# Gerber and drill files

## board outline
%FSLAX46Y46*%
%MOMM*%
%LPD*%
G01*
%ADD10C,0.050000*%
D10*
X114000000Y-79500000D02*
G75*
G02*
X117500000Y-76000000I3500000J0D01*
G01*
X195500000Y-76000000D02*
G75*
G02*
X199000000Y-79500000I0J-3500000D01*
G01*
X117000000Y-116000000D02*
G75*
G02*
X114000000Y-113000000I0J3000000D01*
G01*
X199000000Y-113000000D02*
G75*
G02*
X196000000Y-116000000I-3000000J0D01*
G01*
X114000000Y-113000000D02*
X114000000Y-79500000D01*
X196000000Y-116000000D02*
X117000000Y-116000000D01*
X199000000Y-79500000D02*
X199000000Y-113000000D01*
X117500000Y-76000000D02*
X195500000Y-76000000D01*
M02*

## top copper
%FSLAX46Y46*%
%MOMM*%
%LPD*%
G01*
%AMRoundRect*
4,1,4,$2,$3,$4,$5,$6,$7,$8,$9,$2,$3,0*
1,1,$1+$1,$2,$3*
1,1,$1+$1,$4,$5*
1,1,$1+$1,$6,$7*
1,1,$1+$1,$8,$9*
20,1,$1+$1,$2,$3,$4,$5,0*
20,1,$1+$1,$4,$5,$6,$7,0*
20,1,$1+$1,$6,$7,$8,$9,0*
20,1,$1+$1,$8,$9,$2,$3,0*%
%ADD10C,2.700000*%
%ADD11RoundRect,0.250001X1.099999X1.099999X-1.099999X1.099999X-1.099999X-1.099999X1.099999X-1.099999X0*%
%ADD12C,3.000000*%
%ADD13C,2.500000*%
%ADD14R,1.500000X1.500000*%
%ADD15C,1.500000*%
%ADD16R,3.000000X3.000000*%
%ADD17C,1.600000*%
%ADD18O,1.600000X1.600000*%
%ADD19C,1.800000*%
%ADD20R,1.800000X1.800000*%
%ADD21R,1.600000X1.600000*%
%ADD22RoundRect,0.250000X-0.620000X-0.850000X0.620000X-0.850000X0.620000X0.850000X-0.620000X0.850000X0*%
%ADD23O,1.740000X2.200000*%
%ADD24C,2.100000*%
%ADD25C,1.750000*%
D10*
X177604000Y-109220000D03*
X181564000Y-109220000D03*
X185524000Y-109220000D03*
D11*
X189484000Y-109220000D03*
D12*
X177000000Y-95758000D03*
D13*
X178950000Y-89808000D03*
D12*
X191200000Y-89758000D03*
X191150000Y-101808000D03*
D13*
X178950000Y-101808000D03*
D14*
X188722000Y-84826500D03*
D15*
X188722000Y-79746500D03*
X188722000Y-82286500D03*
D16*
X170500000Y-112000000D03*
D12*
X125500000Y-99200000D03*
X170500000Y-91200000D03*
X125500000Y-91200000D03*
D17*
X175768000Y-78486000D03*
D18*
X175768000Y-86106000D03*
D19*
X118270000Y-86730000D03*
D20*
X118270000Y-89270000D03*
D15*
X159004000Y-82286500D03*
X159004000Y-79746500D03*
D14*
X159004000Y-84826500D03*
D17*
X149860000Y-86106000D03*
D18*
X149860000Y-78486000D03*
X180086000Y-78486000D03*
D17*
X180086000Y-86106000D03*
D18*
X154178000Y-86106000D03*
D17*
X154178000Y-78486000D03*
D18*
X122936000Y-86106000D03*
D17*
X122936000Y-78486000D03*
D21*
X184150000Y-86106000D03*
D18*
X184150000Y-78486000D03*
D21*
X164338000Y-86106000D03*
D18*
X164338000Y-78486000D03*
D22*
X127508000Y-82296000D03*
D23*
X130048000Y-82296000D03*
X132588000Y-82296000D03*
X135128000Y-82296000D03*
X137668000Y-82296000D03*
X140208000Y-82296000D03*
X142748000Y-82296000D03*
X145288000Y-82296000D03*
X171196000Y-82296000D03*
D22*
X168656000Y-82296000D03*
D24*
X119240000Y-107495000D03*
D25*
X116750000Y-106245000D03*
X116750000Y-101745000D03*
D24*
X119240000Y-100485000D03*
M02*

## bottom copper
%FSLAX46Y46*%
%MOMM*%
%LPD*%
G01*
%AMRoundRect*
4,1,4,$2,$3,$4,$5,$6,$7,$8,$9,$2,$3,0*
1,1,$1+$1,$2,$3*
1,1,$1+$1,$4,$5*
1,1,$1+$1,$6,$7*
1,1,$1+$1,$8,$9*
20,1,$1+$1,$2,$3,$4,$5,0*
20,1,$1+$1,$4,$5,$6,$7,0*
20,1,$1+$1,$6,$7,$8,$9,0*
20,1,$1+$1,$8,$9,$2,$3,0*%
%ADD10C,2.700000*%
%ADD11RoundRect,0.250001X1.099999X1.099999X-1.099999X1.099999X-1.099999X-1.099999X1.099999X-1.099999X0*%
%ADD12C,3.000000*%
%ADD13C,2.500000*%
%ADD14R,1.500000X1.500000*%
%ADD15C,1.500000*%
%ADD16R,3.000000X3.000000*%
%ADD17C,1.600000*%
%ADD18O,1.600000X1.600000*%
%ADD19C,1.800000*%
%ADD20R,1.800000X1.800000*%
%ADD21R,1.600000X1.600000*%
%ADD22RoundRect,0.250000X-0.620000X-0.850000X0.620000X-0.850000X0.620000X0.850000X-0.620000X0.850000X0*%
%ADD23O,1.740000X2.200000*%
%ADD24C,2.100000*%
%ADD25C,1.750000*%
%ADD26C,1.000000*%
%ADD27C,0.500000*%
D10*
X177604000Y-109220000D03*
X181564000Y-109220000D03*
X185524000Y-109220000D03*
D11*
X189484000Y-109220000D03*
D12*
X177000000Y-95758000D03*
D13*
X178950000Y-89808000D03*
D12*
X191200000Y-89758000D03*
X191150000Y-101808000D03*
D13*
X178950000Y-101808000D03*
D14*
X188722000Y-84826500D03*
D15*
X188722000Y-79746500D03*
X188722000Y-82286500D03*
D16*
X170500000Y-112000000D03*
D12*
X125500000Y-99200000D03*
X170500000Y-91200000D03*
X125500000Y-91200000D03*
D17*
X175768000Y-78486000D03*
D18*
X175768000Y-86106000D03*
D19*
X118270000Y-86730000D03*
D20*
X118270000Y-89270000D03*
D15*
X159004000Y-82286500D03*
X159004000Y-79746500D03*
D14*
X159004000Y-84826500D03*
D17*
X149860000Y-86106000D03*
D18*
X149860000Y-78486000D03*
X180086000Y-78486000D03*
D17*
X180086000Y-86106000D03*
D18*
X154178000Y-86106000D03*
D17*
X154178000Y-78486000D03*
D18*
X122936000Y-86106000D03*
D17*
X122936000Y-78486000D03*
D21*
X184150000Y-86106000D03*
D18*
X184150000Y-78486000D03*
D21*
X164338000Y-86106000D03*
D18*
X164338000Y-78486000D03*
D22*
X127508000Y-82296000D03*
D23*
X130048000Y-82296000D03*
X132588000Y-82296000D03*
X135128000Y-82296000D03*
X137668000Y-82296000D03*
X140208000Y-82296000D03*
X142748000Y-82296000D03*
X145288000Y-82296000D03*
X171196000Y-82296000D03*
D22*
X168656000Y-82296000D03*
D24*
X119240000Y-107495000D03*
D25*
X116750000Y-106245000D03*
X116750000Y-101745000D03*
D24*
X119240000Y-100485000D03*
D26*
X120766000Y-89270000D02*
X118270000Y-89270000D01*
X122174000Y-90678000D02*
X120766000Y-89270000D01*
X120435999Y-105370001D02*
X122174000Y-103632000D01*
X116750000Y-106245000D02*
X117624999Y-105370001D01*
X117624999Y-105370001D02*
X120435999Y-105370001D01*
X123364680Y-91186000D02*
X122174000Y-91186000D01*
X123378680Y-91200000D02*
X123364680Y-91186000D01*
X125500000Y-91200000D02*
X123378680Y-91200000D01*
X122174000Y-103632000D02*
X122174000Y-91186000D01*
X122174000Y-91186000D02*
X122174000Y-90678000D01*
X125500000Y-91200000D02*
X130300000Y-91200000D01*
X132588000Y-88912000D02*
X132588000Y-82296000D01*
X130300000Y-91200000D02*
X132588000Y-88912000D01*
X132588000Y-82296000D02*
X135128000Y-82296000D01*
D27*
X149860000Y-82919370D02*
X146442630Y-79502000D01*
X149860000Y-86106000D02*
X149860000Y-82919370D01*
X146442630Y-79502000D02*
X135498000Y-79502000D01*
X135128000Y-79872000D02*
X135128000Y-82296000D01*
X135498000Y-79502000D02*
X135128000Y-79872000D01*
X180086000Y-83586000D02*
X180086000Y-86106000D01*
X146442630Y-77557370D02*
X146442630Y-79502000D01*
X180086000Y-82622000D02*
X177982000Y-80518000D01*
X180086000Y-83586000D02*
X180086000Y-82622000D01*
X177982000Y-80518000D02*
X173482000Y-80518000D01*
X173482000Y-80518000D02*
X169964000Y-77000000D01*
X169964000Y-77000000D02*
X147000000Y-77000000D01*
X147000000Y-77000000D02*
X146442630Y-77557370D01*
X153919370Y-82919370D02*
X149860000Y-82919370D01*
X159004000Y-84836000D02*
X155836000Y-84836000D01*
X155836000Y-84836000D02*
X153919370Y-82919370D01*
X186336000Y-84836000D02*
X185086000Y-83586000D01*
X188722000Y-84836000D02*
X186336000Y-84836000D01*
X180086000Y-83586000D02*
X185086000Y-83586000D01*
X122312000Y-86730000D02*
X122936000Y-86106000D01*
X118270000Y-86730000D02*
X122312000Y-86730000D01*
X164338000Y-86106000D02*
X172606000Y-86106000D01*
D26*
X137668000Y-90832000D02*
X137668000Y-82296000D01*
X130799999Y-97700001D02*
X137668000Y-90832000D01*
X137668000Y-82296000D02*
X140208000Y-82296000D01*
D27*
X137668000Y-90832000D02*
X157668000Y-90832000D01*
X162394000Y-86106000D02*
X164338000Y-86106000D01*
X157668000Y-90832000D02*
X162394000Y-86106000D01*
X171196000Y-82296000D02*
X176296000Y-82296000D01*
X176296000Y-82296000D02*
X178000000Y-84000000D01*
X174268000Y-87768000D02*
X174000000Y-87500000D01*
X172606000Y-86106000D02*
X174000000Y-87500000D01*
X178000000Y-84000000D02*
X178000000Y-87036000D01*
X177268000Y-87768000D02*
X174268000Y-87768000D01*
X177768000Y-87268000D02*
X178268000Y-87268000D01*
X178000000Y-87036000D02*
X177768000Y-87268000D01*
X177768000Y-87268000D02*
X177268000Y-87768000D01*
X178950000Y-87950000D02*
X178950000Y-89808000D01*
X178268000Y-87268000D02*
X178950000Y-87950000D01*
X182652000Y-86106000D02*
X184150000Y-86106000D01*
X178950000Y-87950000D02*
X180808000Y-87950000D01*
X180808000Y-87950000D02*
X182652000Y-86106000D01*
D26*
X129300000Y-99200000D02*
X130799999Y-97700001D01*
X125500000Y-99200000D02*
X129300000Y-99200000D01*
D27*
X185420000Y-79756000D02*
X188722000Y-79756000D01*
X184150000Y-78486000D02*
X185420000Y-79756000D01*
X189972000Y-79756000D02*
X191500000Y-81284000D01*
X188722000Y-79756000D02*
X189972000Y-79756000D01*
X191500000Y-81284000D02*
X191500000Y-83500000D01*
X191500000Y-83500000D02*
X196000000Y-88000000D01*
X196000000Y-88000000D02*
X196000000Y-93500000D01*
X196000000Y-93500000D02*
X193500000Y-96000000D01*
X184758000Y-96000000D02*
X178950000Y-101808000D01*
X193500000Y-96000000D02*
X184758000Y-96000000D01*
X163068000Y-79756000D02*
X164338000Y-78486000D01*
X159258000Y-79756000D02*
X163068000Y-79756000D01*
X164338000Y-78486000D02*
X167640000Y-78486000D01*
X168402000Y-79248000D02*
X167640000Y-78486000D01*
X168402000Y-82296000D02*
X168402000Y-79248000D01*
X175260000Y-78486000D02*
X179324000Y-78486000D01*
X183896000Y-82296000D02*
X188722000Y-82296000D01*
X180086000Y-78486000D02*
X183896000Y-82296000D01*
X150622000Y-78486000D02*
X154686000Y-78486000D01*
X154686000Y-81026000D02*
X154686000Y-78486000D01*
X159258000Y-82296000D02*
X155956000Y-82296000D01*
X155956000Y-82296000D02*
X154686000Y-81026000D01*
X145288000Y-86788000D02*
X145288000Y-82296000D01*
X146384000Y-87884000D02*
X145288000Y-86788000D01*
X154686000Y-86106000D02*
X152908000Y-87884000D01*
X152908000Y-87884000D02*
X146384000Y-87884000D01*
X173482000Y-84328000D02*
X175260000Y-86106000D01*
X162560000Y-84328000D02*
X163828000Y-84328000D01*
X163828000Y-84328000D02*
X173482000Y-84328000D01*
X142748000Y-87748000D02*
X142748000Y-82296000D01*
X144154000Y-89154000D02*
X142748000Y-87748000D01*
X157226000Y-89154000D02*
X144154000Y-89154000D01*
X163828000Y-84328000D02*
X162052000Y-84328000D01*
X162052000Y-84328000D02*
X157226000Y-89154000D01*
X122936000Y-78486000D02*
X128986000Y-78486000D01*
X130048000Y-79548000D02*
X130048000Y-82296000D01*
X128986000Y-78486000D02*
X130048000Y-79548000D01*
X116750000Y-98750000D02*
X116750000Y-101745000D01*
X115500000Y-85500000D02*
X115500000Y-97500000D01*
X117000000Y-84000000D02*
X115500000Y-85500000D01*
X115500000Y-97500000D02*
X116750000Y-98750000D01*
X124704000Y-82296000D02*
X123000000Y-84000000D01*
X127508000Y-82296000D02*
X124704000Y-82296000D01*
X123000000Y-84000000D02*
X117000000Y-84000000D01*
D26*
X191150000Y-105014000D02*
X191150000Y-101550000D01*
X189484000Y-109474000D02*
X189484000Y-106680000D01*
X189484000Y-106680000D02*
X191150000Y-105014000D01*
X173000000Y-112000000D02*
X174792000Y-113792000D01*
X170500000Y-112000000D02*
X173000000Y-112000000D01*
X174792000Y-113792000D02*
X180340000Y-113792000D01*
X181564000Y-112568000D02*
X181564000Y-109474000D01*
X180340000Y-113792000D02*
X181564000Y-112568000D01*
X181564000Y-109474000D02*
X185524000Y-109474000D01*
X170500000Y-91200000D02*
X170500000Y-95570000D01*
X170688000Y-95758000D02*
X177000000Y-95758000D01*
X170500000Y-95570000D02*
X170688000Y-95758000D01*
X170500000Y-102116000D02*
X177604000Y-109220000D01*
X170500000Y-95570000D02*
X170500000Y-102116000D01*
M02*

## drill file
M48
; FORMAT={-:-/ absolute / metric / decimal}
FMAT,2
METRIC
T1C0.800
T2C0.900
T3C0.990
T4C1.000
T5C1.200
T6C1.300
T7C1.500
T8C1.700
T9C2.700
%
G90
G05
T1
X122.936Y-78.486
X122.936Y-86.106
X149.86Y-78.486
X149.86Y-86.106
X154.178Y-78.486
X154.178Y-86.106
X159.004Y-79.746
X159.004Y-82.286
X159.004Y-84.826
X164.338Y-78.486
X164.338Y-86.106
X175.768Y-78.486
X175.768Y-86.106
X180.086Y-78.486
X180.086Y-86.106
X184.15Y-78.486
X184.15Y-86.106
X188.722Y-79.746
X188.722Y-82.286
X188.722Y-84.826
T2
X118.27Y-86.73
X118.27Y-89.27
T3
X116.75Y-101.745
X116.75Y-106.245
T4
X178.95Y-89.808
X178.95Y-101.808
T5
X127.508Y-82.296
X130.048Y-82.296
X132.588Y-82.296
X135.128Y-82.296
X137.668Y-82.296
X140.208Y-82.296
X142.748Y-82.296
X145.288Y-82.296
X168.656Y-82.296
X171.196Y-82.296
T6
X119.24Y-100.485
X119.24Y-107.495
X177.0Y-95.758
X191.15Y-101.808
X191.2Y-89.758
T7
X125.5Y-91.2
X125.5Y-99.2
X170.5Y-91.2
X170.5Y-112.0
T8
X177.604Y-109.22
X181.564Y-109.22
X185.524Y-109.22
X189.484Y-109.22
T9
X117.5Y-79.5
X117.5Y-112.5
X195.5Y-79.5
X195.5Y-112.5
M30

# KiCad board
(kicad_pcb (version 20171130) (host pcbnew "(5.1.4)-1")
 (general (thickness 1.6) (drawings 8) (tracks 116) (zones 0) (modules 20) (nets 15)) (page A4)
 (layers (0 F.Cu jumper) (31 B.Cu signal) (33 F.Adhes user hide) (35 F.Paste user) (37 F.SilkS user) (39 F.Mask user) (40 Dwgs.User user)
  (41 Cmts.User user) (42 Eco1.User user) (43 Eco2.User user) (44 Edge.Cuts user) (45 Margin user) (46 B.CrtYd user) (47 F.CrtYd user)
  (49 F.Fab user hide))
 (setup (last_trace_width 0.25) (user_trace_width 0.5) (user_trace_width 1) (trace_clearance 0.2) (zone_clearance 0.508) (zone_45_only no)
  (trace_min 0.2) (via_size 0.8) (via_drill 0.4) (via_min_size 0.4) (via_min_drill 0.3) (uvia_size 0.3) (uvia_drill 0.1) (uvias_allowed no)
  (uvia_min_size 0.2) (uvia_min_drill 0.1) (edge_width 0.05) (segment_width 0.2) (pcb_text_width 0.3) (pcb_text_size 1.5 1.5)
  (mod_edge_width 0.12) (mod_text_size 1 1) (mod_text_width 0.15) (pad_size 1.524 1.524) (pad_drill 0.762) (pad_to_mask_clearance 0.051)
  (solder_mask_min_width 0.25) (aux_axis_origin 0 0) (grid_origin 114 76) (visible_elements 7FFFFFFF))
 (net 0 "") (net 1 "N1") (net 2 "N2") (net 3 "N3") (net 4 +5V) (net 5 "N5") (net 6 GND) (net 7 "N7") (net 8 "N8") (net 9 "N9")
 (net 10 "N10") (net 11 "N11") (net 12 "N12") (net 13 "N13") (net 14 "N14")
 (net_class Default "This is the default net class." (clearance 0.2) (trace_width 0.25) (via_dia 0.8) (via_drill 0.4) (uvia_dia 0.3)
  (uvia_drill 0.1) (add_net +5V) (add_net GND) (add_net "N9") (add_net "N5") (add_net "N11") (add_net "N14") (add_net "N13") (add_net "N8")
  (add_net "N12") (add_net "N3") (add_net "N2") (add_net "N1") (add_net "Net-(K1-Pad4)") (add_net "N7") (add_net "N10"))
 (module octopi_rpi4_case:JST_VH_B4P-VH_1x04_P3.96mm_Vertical (layer F.Cu) (at 189.484 109.22 180)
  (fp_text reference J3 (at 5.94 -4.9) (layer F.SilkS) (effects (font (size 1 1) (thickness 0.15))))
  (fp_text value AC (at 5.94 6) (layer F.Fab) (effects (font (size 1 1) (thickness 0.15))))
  (pad 4 thru_hole circle (at 11.88 0 180) (size 2.7 2.7) (drill 1.7) (layers *.Cu *.Mask) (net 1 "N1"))
  (pad 3 thru_hole circle (at 7.92 0 180) (size 2.7 2.7) (drill 1.7) (layers *.Cu *.Mask) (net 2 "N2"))
  (pad 2 thru_hole circle (at 3.96 0 180) (size 2.7 2.7) (drill 1.7) (layers *.Cu *.Mask) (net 2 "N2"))
  (pad 1 thru_hole roundrect (at 0 0 180) (size 2.7 2.7) (drill 1.7) (layers *.Cu *.Mask) (roundrect_rratio 0.09259299999999999)
   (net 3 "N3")))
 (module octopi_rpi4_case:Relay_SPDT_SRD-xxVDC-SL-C (layer F.Cu) (at 177 95.758)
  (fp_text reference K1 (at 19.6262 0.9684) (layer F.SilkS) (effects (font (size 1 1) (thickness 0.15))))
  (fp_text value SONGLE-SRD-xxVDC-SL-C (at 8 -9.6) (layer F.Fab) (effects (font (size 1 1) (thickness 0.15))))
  (pad 1 thru_hole circle (at 0 0 90) (size 3 3) (drill 1.3) (layers *.Cu *.Mask) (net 1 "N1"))
  (pad 5 thru_hole circle (at 1.95 -5.95 90) (size 2.5 2.5) (drill 1) (layers *.Cu *.Mask) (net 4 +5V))
  (pad 4 thru_hole circle (at 14.2 -6 90) (size 3 3) (drill 1.3) (layers *.Cu *.Mask))
  (pad 3 thru_hole circle (at 14.15 6.05 90) (size 3 3) (drill 1.3) (layers *.Cu *.Mask) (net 3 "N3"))
  (pad 2 thru_hole circle (at 1.95 6.05 90) (size 2.5 2.5) (drill 1) (layers *.Cu *.Mask) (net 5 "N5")))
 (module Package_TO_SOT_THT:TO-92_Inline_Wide (layer F.Cu) (at 188.722 84.8265 90)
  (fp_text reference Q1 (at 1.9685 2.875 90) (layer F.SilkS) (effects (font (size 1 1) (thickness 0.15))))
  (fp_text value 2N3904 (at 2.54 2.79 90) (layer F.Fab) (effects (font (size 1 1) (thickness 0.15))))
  (pad 1 thru_hole rect (at 0 0 180) (size 1.5 1.5) (drill 0.8) (layers *.Cu *.Mask) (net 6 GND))
  (pad 3 thru_hole circle (at 5.08 0 180) (size 1.5 1.5) (drill 0.8) (layers *.Cu *.Mask) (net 5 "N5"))
  (pad 2 thru_hole circle (at 2.54 0 180) (size 1.5 1.5) (drill 0.8) (layers *.Cu *.Mask) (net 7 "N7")))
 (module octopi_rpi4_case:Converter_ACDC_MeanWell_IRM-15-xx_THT (layer F.Cu) (at 170.5 112 180)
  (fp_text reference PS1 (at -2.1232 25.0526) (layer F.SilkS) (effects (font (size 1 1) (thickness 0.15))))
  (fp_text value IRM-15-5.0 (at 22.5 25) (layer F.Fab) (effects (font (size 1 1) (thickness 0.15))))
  (pad 1 thru_hole rect (at 0 0 180) (size 3 3) (drill 1.5) (layers *.Cu *.Mask) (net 2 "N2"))
  (pad 4 thru_hole circle (at 45 12.8 180) (size 3 3) (drill 1.5) (layers *.Cu *.Mask) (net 4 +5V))
  (pad 2 thru_hole circle (at 0 20.8 180) (size 3 3) (drill 1.5) (layers *.Cu *.Mask) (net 1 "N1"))
  (pad 3 thru_hole circle (at 45 20.8 180) (size 3 3) (drill 1.5) (layers *.Cu *.Mask) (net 6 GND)))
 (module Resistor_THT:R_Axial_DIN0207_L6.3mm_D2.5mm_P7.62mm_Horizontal (layer F.Cu) (at 175.768 78.486 270)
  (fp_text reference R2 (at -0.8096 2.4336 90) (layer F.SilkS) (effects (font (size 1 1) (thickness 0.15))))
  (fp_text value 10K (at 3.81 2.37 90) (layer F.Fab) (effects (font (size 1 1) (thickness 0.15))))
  (pad 1 thru_hole circle (at 0 0 270) (size 1.6 1.6) (drill 0.8) (layers *.Cu *.Mask) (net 7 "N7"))
  (pad 2 thru_hole oval (at 7.62 0 270) (size 1.6 1.6) (drill 0.8) (layers *.Cu *.Mask) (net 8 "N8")))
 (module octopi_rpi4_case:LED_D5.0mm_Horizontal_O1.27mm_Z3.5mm (layer F.Cu) (at 118.27 86.73 270)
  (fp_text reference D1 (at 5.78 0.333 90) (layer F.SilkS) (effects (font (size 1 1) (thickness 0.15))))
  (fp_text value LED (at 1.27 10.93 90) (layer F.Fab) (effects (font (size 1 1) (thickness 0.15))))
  (pad 2 thru_hole circle (at 0 0 270) (size 1.8 1.8) (drill 0.9) (layers *.Cu *.Mask) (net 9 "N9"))
  (pad 1 thru_hole rect (at 2.54 0 270) (size 1.8 1.8) (drill 0.9) (layers *.Cu *.Mask) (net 6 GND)))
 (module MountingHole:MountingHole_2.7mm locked (layer F.Cu) (at 195.5 79.5)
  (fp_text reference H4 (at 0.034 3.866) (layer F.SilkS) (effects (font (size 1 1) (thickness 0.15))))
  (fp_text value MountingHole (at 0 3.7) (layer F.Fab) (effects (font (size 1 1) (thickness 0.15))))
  (pad 1 np_thru_hole circle (at 0 0) (size 2.7 2.7) (drill 2.7) (layers *.Cu *.Mask)))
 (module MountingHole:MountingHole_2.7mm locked (layer F.Cu) (at 117.5 79.5)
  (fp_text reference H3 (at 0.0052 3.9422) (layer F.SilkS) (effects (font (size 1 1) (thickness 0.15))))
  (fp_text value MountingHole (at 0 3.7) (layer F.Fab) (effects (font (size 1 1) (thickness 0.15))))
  (pad 1 np_thru_hole circle (at 0 0) (size 2.7 2.7) (drill 2.7) (layers *.Cu *.Mask)))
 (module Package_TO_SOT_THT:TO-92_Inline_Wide (layer F.Cu) (at 159.004 84.8265 90)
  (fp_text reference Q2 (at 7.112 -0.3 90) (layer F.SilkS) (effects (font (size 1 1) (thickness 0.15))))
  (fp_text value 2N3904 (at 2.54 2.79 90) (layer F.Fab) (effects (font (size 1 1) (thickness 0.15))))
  (pad 2 thru_hole circle (at 2.54 0 180) (size 1.5 1.5) (drill 0.8) (layers *.Cu *.Mask) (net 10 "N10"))
  (pad 3 thru_hole circle (at 5.08 0 180) (size 1.5 1.5) (drill 0.8) (layers *.Cu *.Mask) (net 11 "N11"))
  (pad 1 thru_hole rect (at 0 0 180) (size 1.5 1.5) (drill 0.8) (layers *.Cu *.Mask) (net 6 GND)))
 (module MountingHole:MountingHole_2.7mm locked (layer F.Cu) (at 195.5 112.5)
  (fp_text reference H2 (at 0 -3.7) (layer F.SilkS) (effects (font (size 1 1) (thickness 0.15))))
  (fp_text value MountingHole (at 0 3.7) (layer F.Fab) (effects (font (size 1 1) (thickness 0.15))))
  (pad 1 np_thru_hole circle (at 0 0) (size 2.7 2.7) (drill 2.7) (layers *.Cu *.Mask)))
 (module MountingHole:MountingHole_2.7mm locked (layer F.Cu) (at 117.5 112.5)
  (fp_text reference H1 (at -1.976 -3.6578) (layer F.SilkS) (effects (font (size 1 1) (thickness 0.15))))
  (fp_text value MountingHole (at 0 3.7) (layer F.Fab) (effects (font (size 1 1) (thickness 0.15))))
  (pad 1 np_thru_hole circle (at 0 0) (size 2.7 2.7) (drill 2.7) (layers *.Cu *.Mask)))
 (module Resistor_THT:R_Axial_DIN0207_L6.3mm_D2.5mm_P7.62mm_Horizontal (layer F.Cu) (at 149.86 86.106 90)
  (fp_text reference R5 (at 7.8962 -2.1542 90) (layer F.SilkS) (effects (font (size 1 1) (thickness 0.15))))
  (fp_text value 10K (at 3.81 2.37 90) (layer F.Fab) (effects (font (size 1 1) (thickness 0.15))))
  (pad 1 thru_hole circle (at 0 0 90) (size 1.6 1.6) (drill 0.8) (layers *.Cu *.Mask) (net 6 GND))
  (pad 2 thru_hole oval (at 7.62 0 90) (size 1.6 1.6) (drill 0.8) (layers *.Cu *.Mask) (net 10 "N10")))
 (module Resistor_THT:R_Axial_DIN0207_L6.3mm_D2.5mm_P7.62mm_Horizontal (layer F.Cu) (at 180.086 86.106 90)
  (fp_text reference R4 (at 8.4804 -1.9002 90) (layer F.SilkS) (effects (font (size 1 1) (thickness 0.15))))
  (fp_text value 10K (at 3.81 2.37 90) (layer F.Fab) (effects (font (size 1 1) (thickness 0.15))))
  (pad 2 thru_hole oval (at 7.62 0 90) (size 1.6 1.6) (drill 0.8) (layers *.Cu *.Mask) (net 7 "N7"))
  (pad 1 thru_hole circle (at 0 0 90) (size 1.6 1.6) (drill 0.8) (layers *.Cu *.Mask) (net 6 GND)))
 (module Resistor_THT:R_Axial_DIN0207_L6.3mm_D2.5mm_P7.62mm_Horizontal (layer F.Cu) (at 154.178 78.486 270)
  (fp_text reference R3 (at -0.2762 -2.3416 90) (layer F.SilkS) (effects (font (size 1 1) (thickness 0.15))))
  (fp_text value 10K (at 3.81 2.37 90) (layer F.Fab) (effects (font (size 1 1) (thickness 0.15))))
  (pad 2 thru_hole oval (at 7.62 0 270) (size 1.6 1.6) (drill 0.8) (layers *.Cu *.Mask) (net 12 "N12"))
  (pad 1 thru_hole circle (at 0 0 270) (size 1.6 1.6) (drill 0.8) (layers *.Cu *.Mask) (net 10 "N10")))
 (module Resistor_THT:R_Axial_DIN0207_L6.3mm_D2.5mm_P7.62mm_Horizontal (layer F.Cu) (at 122.936 78.486 270)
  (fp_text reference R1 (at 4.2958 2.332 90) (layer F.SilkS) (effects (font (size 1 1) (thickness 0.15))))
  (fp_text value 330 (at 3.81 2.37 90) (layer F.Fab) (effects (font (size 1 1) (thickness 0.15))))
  (pad 2 thru_hole oval (at 7.62 0 270) (size 1.6 1.6) (drill 0.8) (layers *.Cu *.Mask) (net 9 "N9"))
  (pad 1 thru_hole circle (at 0 0 270) (size 1.6 1.6) (drill 0.8) (layers *.Cu *.Mask) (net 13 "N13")))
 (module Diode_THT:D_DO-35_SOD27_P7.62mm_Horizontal (layer F.Cu) (at 184.15 86.106 90)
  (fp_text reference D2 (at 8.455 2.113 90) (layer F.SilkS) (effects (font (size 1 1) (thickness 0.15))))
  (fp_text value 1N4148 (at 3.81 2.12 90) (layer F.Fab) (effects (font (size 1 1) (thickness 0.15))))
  (pad 1 thru_hole rect (at 0 0 90) (size 1.6 1.6) (drill 0.8) (layers *.Cu *.Mask) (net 4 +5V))
  (pad 2 thru_hole oval (at 7.62 0 90) (size 1.6 1.6) (drill 0.8) (layers *.Cu *.Mask) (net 5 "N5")))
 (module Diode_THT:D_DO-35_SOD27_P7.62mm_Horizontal (layer F.Cu) (at 164.338 86.106 90)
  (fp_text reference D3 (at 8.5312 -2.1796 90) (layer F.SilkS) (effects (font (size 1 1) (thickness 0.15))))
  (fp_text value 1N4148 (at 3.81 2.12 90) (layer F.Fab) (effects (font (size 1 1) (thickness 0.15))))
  (pad 1 thru_hole rect (at 0 0 90) (size 1.6 1.6) (drill 0.8) (layers *.Cu *.Mask) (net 4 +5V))
  (pad 2 thru_hole oval (at 7.62 0 90) (size 1.6 1.6) (drill 0.8) (layers *.Cu *.Mask) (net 11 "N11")))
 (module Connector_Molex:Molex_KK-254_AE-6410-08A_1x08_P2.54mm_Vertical (layer F.Cu) (at 127.508 82.296)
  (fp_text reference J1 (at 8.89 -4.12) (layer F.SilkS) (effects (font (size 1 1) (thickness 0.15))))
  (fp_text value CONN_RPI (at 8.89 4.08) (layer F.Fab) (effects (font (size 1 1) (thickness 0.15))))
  (pad 1 thru_hole roundrect (at 0 0) (size 1.74 2.2) (drill 1.2) (layers *.Cu *.Mask) (roundrect_rratio 0.143678) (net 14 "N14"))
  (pad 2 thru_hole oval (at 2.54 0) (size 1.74 2.2) (drill 1.2) (layers *.Cu *.Mask) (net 13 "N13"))
  (pad 3 thru_hole oval (at 5.08 0) (size 1.74 2.2) (drill 1.2) (layers *.Cu *.Mask) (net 6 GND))
  (pad 4 thru_hole oval (at 7.62 0) (size 1.74 2.2) (drill 1.2) (layers *.Cu *.Mask) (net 6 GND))
  (pad 5 thru_hole oval (at 10.16 0) (size 1.74 2.2) (drill 1.2) (layers *.Cu *.Mask) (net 4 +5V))
  (pad 6 thru_hole oval (at 12.7 0) (size 1.74 2.2) (drill 1.2) (layers *.Cu *.Mask) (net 4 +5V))
  (pad 7 thru_hole oval (at 15.24 0) (size 1.74 2.2) (drill 1.2) (layers *.Cu *.Mask) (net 8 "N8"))
  (pad 8 thru_hole oval (at 17.78 0) (size 1.74 2.2) (drill 1.2) (layers *.Cu *.Mask) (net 12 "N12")))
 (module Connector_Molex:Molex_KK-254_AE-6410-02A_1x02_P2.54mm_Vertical (layer F.Cu) (at 168.656 82.296)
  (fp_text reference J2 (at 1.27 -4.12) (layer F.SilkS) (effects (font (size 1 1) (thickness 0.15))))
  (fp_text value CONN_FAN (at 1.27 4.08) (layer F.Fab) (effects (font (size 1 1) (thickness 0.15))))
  (pad 2 thru_hole oval (at 2.54 0) (size 1.74 2.2) (drill 1.2) (layers *.Cu *.Mask) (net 4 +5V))
  (pad 1 thru_hole roundrect (at 0 0) (size 1.74 2.2) (drill 1.2) (layers *.Cu *.Mask) (roundrect_rratio 0.143678) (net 11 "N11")))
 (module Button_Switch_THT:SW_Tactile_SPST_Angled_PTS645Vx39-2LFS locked (layer F.Cu) (at 116.75 106.245 90)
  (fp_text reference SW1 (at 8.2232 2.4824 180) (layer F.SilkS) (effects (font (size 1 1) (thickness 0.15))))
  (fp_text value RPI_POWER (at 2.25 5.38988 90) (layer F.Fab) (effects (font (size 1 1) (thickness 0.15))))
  (pad "" thru_hole circle (at -1.25 2.49 90) (size 2.1 2.1) (drill 1.3) (layers *.Cu *.Mask))
  (pad 1 thru_hole circle (at 0 0 90) (size 1.75 1.75) (drill 0.99) (layers *.Cu *.Mask) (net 6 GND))
  (pad 2 thru_hole circle (at 4.5 0 90) (size 1.75 1.75) (drill 0.99) (layers *.Cu *.Mask) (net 14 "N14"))
  (pad "" thru_hole circle (at 5.76 2.49 90) (size 2.1 2.1) (drill 1.3) (layers *.Cu *.Mask)))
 (gr_arc (start 117.5 79.5) (end 117.5 76) (angle -90) (layer Edge.Cuts) (width 0.05))
 (gr_arc (start 195.5 79.5) (end 199 79.5) (angle -90) (layer Edge.Cuts) (width 0.05))
 (gr_arc (start 117 113) (end 114 113) (angle -90) (layer Edge.Cuts) (width 0.05))
 (gr_arc (start 196 113) (end 196 116) (angle -90) (layer Edge.Cuts) (width 0.05))
 (gr_line (start 114 113) (end 114 79.5) (layer Edge.Cuts) (width 0.05))
 (gr_line (start 196 116) (end 117 116) (layer Edge.Cuts) (width 0.05))
 (gr_line (start 199 79.5) (end 199 113) (layer Edge.Cuts) (width 0.05))
 (gr_line (start 117.5 76) (end 195.5 76) (layer Edge.Cuts) (width 0.05))
 (segment (start 120.766 89.27) (end 118.27 89.27) (width 1) (layer B.Cu) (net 6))
 (segment (start 122.174 90.678) (end 120.766 89.27) (width 1) (layer B.Cu) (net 6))
 (segment (start 120.435999 105.370001) (end 122.174 103.632) (width 1) (layer B.Cu) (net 6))
 (segment (start 116.75 106.245) (end 117.624999 105.370001) (width 1) (layer B.Cu) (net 6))
 (segment (start 117.624999 105.370001) (end 120.435999 105.370001) (width 1) (layer B.Cu) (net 6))
 (segment (start 123.36468 91.186) (end 122.174 91.186) (width 1) (layer B.Cu) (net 6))
 (segment (start 123.37868 91.2) (end 123.36468 91.186) (width 1) (layer B.Cu) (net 6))
 (segment (start 125.5 91.2) (end 123.37868 91.2) (width 1) (layer B.Cu) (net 6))
 (segment (start 122.174 103.632) (end 122.174 91.186) (width 1) (layer B.Cu) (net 6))
 (segment (start 122.174 91.186) (end 122.174 90.678) (width 1) (layer B.Cu) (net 6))
 (segment (start 125.5 91.2) (end 130.3 91.2) (width 1) (layer B.Cu) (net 6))
 (segment (start 132.588 88.912) (end 132.588 82.296) (width 1) (layer B.Cu) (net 6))
 (segment (start 130.3 91.2) (end 132.588 88.912) (width 1) (layer B.Cu) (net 6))
 (segment (start 132.588 82.296) (end 135.128 82.296) (width 1) (layer B.Cu) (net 6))
 (segment (start 149.86 82.91937) (end 146.44263 79.502) (width 0.5) (layer B.Cu) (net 6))
 (segment (start 149.86 86.106) (end 149.86 82.91937) (width 0.5) (layer B.Cu) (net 6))
 (segment (start 146.44263 79.502) (end 135.498 79.502) (width 0.5) (layer B.Cu) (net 6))
 (segment (start 135.128 79.872) (end 135.128 82.296) (width 0.5) (layer B.Cu) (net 6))
 (segment (start 135.498 79.502) (end 135.128 79.872) (width 0.5) (layer B.Cu) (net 6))
 (segment (start 180.086 83.586) (end 180.086 86.106) (width 0.5) (layer B.Cu) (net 6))
 (segment (start 146.44263 77.55737) (end 146.44263 79.502) (width 0.5) (layer B.Cu) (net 6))
 (segment (start 180.086 82.622) (end 177.982 80.518) (width 0.5) (layer B.Cu) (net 6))
 (segment (start 180.086 83.586) (end 180.086 82.622) (width 0.5) (layer B.Cu) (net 6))
 (segment (start 177.982 80.518) (end 173.482 80.518) (width 0.5) (layer B.Cu) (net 6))
 (segment (start 173.482 80.518) (end 169.964 77) (width 0.5) (layer B.Cu) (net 6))
 (segment (start 169.964 77) (end 147 77) (width 0.5) (layer B.Cu) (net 6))
 (segment (start 147 77) (end 146.44263 77.55737) (width 0.5) (layer B.Cu) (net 6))
 (segment (start 153.91937 82.91937) (end 149.86 82.91937) (width 0.5) (layer B.Cu) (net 6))
 (segment (start 159.004 84.836) (end 155.836 84.836) (width 0.5) (layer B.Cu) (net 6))
 (segment (start 155.836 84.836) (end 153.91937 82.91937) (width 0.5) (layer B.Cu) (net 6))
 (segment (start 186.336 84.836) (end 185.086 83.586) (width 0.5) (layer B.Cu) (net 6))
 (segment (start 188.722 84.836) (end 186.336 84.836) (width 0.5) (layer B.Cu) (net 6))
 (segment (start 180.086 83.586) (end 185.086 83.586) (width 0.5) (layer B.Cu) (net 6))
 (segment (start 122.312 86.73) (end 122.936 86.106) (width 0.5) (layer B.Cu) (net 9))
 (segment (start 118.27 86.73) (end 122.312 86.73) (width 0.5) (layer B.Cu) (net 9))
 (segment (start 164.338 86.106) (end 172.606 86.106) (width 0.5) (layer B.Cu) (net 4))
 (segment (start 137.668 90.832) (end 137.668 82.296) (width 1) (layer B.Cu) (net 4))
 (segment (start 130.799999 97.700001) (end 137.668 90.832) (width 1) (layer B.Cu) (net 4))
 (segment (start 137.668 82.296) (end 140.208 82.296) (width 1) (layer B.Cu) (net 4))
 (segment (start 137.668 90.832) (end 157.668 90.832) (width 0.5) (layer B.Cu) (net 4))
 (segment (start 162.394 86.106) (end 164.338 86.106) (width 0.5) (layer B.Cu) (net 4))
 (segment (start 157.668 90.832) (end 162.394 86.106) (width 0.5) (layer B.Cu) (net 4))
 (segment (start 171.196 82.296) (end 176.296 82.296) (width 0.5) (layer B.Cu) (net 4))
 (segment (start 176.296 82.296) (end 178 84) (width 0.5) (layer B.Cu) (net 4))
 (segment (start 174.268 87.768) (end 174 87.5) (width 0.5) (layer B.Cu) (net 4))
 (segment (start 172.606 86.106) (end 174 87.5) (width 0.5) (layer B.Cu) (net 4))
 (segment (start 178 84) (end 178 87.036) (width 0.5) (layer B.Cu) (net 4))
 (segment (start 177.268 87.768) (end 174.268 87.768) (width 0.5) (layer B.Cu) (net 4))
 (segment (start 177.768 87.268) (end 178.268 87.268) (width 0.5) (layer B.Cu) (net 4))
 (segment (start 178 87.036) (end 177.768 87.268) (width 0.5) (layer B.Cu) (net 4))
 (segment (start 177.768 87.268) (end 177.268 87.768) (width 0.5) (layer B.Cu) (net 4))
 (segment (start 178.95 87.95) (end 178.95 89.808) (width 0.5) (layer B.Cu) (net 4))
 (segment (start 178.268 87.268) (end 178.95 87.95) (width 0.5) (layer B.Cu) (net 4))
 (segment (start 182.652 86.106) (end 184.15 86.106) (width 0.5) (layer B.Cu) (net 4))
 (segment (start 178.95 87.95) (end 180.808 87.95) (width 0.5) (layer B.Cu) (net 4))
 (segment (start 180.808 87.95) (end 182.652 86.106) (width 0.5) (layer B.Cu) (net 4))
 (segment (start 129.3 99.2) (end 130.799999 97.700001) (width 1) (layer B.Cu) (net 4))
 (segment (start 125.5 99.2) (end 129.3 99.2) (width 1) (layer B.Cu) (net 4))
 (segment (start 185.42 79.756) (end 188.722 79.756) (width 0.5) (layer B.Cu) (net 5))
 (segment (start 184.15 78.486) (end 185.42 79.756) (width 0.5) (layer B.Cu) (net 5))
 (segment (start 189.972 79.756) (end 191.5 81.284) (width 0.5) (layer B.Cu) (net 5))
 (segment (start 188.722 79.756) (end 189.972 79.756) (width 0.5) (layer B.Cu) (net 5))
 (segment (start 191.5 81.284) (end 191.5 83.5) (width 0.5) (layer B.Cu) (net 5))
 (segment (start 191.5 83.5) (end 196 88) (width 0.5) (layer B.Cu) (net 5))
 (segment (start 196 88) (end 196 93.5) (width 0.5) (layer B.Cu) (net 5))
 (segment (start 196 93.5) (end 193.5 96) (width 0.5) (layer B.Cu) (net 5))
 (segment (start 184.758 96) (end 178.95 101.808) (width 0.5) (layer B.Cu) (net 5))
 (segment (start 193.5 96) (end 184.758 96) (width 0.5) (layer B.Cu) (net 5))
 (segment (start 163.068 79.756) (end 164.338 78.486) (width 0.5) (layer B.Cu) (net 11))
 (segment (start 159.258 79.756) (end 163.068 79.756) (width 0.5) (layer B.Cu) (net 11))
 (segment (start 164.338 78.486) (end 167.64 78.486) (width 0.5) (layer B.Cu) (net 11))
 (segment (start 168.402 79.248) (end 167.64 78.486) (width 0.5) (layer B.Cu) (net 11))
 (segment (start 168.402 82.296) (end 168.402 79.248) (width 0.5) (layer B.Cu) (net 11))
 (segment (start 175.26 78.486) (end 179.324 78.486) (width 0.5) (layer B.Cu) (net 7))
 (segment (start 183.896 82.296) (end 188.722 82.296) (width 0.5) (layer B.Cu) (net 7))
 (segment (start 180.086 78.486) (end 183.896 82.296) (width 0.5) (layer B.Cu) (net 7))
 (segment (start 150.622 78.486) (end 154.686 78.486) (width 0.5) (layer B.Cu) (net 10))
 (segment (start 154.686 81.026) (end 154.686 78.486) (width 0.5) (layer B.Cu) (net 10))
 (segment (start 159.258 82.296) (end 155.956 82.296) (width 0.5) (layer B.Cu) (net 10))
 (segment (start 155.956 82.296) (end 154.686 81.026) (width 0.5) (layer B.Cu) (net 10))
 (segment (start 145.288 86.788) (end 145.288 82.296) (width 0.5) (layer B.Cu) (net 12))
 (segment (start 146.384 87.884) (end 145.288 86.788) (width 0.5) (layer B.Cu) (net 12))
 (segment (start 154.686 86.106) (end 152.908 87.884) (width 0.5) (layer B.Cu) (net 12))
 (segment (start 152.908 87.884) (end 146.384 87.884) (width 0.5) (layer B.Cu) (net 12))
 (segment (start 173.482 84.328) (end 175.26 86.106) (width 0.5) (layer B.Cu) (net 8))
 (segment (start 162.56 84.328) (end 163.828 84.328) (width 0.5) (layer B.Cu) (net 8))
 (segment (start 163.828 84.328) (end 173.482 84.328) (width 0.5) (layer B.Cu) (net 8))
 (segment (start 142.748 87.748) (end 142.748 82.296) (width 0.5) (layer B.Cu) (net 8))
 (segment (start 144.154 89.154) (end 142.748 87.748) (width 0.5) (layer B.Cu) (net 8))
 (segment (start 157.226 89.154) (end 144.154 89.154) (width 0.5) (layer B.Cu) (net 8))
 (segment (start 163.828 84.328) (end 162.052 84.328) (width 0.5) (layer B.Cu) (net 8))
 (segment (start 162.052 84.328) (end 157.226 89.154) (width 0.5) (layer B.Cu) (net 8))
 (segment (start 122.936 78.486) (end 128.986 78.486) (width 0.5) (layer B.Cu) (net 13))
 (segment (start 130.048 79.548) (end 130.048 82.296) (width 0.5) (layer B.Cu) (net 13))
 (segment (start 128.986 78.486) (end 130.048 79.548) (width 0.5) (layer B.Cu) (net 13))
 (segment (start 116.75 98.75) (end 116.75 101.745) (width 0.5) (layer B.Cu) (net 14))
 (segment (start 115.5 85.5) (end 115.5 97.5) (width 0.5) (layer B.Cu) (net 14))
 (segment (start 117 84) (end 115.5 85.5) (width 0.5) (layer B.Cu) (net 14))
 (segment (start 115.5 97.5) (end 116.75 98.75) (width 0.5) (layer B.Cu) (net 14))
 (segment (start 124.704 82.296) (end 123 84) (width 0.5) (layer B.Cu) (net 14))
 (segment (start 127.508 82.296) (end 124.704 82.296) (width 0.5) (layer B.Cu) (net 14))
 (segment (start 123 84) (end 117 84) (width 0.5) (layer B.Cu) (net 14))
 (segment (start 191.15 105.014) (end 191.15 101.55) (width 1) (layer B.Cu) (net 3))
 (segment (start 189.484 109.474) (end 189.484 106.68) (width 1) (layer B.Cu) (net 3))
 (segment (start 189.484 106.68) (end 191.15 105.014) (width 1) (layer B.Cu) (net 3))
 (segment (start 173 112) (end 174.792 113.792) (width 1) (layer B.Cu) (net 2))
 (segment (start 170.5 112) (end 173 112) (width 1) (layer B.Cu) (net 2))
 (segment (start 174.792 113.792) (end 180.34 113.792) (width 1) (layer B.Cu) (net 2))
 (segment (start 181.564 112.568) (end 181.564 109.474) (width 1) (layer B.Cu) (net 2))
 (segment (start 180.34 113.792) (end 181.564 112.568) (width 1) (layer B.Cu) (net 2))
 (segment (start 181.564 109.474) (end 185.524 109.474) (width 1) (layer B.Cu) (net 2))
 (segment (start 170.5 91.2) (end 170.5 95.57) (width 1) (layer B.Cu) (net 1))
 (segment (start 170.688 95.758) (end 177 95.758) (width 1) (layer B.Cu) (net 1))
 (segment (start 170.5 95.57) (end 170.688 95.758) (width 1) (layer B.Cu) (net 1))
 (segment (start 170.5 102.116) (end 177.604 109.22) (width 1) (layer B.Cu) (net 1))
 (segment (start 170.5 95.57) (end 170.5 102.116) (width 1) (layer B.Cu) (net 1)))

